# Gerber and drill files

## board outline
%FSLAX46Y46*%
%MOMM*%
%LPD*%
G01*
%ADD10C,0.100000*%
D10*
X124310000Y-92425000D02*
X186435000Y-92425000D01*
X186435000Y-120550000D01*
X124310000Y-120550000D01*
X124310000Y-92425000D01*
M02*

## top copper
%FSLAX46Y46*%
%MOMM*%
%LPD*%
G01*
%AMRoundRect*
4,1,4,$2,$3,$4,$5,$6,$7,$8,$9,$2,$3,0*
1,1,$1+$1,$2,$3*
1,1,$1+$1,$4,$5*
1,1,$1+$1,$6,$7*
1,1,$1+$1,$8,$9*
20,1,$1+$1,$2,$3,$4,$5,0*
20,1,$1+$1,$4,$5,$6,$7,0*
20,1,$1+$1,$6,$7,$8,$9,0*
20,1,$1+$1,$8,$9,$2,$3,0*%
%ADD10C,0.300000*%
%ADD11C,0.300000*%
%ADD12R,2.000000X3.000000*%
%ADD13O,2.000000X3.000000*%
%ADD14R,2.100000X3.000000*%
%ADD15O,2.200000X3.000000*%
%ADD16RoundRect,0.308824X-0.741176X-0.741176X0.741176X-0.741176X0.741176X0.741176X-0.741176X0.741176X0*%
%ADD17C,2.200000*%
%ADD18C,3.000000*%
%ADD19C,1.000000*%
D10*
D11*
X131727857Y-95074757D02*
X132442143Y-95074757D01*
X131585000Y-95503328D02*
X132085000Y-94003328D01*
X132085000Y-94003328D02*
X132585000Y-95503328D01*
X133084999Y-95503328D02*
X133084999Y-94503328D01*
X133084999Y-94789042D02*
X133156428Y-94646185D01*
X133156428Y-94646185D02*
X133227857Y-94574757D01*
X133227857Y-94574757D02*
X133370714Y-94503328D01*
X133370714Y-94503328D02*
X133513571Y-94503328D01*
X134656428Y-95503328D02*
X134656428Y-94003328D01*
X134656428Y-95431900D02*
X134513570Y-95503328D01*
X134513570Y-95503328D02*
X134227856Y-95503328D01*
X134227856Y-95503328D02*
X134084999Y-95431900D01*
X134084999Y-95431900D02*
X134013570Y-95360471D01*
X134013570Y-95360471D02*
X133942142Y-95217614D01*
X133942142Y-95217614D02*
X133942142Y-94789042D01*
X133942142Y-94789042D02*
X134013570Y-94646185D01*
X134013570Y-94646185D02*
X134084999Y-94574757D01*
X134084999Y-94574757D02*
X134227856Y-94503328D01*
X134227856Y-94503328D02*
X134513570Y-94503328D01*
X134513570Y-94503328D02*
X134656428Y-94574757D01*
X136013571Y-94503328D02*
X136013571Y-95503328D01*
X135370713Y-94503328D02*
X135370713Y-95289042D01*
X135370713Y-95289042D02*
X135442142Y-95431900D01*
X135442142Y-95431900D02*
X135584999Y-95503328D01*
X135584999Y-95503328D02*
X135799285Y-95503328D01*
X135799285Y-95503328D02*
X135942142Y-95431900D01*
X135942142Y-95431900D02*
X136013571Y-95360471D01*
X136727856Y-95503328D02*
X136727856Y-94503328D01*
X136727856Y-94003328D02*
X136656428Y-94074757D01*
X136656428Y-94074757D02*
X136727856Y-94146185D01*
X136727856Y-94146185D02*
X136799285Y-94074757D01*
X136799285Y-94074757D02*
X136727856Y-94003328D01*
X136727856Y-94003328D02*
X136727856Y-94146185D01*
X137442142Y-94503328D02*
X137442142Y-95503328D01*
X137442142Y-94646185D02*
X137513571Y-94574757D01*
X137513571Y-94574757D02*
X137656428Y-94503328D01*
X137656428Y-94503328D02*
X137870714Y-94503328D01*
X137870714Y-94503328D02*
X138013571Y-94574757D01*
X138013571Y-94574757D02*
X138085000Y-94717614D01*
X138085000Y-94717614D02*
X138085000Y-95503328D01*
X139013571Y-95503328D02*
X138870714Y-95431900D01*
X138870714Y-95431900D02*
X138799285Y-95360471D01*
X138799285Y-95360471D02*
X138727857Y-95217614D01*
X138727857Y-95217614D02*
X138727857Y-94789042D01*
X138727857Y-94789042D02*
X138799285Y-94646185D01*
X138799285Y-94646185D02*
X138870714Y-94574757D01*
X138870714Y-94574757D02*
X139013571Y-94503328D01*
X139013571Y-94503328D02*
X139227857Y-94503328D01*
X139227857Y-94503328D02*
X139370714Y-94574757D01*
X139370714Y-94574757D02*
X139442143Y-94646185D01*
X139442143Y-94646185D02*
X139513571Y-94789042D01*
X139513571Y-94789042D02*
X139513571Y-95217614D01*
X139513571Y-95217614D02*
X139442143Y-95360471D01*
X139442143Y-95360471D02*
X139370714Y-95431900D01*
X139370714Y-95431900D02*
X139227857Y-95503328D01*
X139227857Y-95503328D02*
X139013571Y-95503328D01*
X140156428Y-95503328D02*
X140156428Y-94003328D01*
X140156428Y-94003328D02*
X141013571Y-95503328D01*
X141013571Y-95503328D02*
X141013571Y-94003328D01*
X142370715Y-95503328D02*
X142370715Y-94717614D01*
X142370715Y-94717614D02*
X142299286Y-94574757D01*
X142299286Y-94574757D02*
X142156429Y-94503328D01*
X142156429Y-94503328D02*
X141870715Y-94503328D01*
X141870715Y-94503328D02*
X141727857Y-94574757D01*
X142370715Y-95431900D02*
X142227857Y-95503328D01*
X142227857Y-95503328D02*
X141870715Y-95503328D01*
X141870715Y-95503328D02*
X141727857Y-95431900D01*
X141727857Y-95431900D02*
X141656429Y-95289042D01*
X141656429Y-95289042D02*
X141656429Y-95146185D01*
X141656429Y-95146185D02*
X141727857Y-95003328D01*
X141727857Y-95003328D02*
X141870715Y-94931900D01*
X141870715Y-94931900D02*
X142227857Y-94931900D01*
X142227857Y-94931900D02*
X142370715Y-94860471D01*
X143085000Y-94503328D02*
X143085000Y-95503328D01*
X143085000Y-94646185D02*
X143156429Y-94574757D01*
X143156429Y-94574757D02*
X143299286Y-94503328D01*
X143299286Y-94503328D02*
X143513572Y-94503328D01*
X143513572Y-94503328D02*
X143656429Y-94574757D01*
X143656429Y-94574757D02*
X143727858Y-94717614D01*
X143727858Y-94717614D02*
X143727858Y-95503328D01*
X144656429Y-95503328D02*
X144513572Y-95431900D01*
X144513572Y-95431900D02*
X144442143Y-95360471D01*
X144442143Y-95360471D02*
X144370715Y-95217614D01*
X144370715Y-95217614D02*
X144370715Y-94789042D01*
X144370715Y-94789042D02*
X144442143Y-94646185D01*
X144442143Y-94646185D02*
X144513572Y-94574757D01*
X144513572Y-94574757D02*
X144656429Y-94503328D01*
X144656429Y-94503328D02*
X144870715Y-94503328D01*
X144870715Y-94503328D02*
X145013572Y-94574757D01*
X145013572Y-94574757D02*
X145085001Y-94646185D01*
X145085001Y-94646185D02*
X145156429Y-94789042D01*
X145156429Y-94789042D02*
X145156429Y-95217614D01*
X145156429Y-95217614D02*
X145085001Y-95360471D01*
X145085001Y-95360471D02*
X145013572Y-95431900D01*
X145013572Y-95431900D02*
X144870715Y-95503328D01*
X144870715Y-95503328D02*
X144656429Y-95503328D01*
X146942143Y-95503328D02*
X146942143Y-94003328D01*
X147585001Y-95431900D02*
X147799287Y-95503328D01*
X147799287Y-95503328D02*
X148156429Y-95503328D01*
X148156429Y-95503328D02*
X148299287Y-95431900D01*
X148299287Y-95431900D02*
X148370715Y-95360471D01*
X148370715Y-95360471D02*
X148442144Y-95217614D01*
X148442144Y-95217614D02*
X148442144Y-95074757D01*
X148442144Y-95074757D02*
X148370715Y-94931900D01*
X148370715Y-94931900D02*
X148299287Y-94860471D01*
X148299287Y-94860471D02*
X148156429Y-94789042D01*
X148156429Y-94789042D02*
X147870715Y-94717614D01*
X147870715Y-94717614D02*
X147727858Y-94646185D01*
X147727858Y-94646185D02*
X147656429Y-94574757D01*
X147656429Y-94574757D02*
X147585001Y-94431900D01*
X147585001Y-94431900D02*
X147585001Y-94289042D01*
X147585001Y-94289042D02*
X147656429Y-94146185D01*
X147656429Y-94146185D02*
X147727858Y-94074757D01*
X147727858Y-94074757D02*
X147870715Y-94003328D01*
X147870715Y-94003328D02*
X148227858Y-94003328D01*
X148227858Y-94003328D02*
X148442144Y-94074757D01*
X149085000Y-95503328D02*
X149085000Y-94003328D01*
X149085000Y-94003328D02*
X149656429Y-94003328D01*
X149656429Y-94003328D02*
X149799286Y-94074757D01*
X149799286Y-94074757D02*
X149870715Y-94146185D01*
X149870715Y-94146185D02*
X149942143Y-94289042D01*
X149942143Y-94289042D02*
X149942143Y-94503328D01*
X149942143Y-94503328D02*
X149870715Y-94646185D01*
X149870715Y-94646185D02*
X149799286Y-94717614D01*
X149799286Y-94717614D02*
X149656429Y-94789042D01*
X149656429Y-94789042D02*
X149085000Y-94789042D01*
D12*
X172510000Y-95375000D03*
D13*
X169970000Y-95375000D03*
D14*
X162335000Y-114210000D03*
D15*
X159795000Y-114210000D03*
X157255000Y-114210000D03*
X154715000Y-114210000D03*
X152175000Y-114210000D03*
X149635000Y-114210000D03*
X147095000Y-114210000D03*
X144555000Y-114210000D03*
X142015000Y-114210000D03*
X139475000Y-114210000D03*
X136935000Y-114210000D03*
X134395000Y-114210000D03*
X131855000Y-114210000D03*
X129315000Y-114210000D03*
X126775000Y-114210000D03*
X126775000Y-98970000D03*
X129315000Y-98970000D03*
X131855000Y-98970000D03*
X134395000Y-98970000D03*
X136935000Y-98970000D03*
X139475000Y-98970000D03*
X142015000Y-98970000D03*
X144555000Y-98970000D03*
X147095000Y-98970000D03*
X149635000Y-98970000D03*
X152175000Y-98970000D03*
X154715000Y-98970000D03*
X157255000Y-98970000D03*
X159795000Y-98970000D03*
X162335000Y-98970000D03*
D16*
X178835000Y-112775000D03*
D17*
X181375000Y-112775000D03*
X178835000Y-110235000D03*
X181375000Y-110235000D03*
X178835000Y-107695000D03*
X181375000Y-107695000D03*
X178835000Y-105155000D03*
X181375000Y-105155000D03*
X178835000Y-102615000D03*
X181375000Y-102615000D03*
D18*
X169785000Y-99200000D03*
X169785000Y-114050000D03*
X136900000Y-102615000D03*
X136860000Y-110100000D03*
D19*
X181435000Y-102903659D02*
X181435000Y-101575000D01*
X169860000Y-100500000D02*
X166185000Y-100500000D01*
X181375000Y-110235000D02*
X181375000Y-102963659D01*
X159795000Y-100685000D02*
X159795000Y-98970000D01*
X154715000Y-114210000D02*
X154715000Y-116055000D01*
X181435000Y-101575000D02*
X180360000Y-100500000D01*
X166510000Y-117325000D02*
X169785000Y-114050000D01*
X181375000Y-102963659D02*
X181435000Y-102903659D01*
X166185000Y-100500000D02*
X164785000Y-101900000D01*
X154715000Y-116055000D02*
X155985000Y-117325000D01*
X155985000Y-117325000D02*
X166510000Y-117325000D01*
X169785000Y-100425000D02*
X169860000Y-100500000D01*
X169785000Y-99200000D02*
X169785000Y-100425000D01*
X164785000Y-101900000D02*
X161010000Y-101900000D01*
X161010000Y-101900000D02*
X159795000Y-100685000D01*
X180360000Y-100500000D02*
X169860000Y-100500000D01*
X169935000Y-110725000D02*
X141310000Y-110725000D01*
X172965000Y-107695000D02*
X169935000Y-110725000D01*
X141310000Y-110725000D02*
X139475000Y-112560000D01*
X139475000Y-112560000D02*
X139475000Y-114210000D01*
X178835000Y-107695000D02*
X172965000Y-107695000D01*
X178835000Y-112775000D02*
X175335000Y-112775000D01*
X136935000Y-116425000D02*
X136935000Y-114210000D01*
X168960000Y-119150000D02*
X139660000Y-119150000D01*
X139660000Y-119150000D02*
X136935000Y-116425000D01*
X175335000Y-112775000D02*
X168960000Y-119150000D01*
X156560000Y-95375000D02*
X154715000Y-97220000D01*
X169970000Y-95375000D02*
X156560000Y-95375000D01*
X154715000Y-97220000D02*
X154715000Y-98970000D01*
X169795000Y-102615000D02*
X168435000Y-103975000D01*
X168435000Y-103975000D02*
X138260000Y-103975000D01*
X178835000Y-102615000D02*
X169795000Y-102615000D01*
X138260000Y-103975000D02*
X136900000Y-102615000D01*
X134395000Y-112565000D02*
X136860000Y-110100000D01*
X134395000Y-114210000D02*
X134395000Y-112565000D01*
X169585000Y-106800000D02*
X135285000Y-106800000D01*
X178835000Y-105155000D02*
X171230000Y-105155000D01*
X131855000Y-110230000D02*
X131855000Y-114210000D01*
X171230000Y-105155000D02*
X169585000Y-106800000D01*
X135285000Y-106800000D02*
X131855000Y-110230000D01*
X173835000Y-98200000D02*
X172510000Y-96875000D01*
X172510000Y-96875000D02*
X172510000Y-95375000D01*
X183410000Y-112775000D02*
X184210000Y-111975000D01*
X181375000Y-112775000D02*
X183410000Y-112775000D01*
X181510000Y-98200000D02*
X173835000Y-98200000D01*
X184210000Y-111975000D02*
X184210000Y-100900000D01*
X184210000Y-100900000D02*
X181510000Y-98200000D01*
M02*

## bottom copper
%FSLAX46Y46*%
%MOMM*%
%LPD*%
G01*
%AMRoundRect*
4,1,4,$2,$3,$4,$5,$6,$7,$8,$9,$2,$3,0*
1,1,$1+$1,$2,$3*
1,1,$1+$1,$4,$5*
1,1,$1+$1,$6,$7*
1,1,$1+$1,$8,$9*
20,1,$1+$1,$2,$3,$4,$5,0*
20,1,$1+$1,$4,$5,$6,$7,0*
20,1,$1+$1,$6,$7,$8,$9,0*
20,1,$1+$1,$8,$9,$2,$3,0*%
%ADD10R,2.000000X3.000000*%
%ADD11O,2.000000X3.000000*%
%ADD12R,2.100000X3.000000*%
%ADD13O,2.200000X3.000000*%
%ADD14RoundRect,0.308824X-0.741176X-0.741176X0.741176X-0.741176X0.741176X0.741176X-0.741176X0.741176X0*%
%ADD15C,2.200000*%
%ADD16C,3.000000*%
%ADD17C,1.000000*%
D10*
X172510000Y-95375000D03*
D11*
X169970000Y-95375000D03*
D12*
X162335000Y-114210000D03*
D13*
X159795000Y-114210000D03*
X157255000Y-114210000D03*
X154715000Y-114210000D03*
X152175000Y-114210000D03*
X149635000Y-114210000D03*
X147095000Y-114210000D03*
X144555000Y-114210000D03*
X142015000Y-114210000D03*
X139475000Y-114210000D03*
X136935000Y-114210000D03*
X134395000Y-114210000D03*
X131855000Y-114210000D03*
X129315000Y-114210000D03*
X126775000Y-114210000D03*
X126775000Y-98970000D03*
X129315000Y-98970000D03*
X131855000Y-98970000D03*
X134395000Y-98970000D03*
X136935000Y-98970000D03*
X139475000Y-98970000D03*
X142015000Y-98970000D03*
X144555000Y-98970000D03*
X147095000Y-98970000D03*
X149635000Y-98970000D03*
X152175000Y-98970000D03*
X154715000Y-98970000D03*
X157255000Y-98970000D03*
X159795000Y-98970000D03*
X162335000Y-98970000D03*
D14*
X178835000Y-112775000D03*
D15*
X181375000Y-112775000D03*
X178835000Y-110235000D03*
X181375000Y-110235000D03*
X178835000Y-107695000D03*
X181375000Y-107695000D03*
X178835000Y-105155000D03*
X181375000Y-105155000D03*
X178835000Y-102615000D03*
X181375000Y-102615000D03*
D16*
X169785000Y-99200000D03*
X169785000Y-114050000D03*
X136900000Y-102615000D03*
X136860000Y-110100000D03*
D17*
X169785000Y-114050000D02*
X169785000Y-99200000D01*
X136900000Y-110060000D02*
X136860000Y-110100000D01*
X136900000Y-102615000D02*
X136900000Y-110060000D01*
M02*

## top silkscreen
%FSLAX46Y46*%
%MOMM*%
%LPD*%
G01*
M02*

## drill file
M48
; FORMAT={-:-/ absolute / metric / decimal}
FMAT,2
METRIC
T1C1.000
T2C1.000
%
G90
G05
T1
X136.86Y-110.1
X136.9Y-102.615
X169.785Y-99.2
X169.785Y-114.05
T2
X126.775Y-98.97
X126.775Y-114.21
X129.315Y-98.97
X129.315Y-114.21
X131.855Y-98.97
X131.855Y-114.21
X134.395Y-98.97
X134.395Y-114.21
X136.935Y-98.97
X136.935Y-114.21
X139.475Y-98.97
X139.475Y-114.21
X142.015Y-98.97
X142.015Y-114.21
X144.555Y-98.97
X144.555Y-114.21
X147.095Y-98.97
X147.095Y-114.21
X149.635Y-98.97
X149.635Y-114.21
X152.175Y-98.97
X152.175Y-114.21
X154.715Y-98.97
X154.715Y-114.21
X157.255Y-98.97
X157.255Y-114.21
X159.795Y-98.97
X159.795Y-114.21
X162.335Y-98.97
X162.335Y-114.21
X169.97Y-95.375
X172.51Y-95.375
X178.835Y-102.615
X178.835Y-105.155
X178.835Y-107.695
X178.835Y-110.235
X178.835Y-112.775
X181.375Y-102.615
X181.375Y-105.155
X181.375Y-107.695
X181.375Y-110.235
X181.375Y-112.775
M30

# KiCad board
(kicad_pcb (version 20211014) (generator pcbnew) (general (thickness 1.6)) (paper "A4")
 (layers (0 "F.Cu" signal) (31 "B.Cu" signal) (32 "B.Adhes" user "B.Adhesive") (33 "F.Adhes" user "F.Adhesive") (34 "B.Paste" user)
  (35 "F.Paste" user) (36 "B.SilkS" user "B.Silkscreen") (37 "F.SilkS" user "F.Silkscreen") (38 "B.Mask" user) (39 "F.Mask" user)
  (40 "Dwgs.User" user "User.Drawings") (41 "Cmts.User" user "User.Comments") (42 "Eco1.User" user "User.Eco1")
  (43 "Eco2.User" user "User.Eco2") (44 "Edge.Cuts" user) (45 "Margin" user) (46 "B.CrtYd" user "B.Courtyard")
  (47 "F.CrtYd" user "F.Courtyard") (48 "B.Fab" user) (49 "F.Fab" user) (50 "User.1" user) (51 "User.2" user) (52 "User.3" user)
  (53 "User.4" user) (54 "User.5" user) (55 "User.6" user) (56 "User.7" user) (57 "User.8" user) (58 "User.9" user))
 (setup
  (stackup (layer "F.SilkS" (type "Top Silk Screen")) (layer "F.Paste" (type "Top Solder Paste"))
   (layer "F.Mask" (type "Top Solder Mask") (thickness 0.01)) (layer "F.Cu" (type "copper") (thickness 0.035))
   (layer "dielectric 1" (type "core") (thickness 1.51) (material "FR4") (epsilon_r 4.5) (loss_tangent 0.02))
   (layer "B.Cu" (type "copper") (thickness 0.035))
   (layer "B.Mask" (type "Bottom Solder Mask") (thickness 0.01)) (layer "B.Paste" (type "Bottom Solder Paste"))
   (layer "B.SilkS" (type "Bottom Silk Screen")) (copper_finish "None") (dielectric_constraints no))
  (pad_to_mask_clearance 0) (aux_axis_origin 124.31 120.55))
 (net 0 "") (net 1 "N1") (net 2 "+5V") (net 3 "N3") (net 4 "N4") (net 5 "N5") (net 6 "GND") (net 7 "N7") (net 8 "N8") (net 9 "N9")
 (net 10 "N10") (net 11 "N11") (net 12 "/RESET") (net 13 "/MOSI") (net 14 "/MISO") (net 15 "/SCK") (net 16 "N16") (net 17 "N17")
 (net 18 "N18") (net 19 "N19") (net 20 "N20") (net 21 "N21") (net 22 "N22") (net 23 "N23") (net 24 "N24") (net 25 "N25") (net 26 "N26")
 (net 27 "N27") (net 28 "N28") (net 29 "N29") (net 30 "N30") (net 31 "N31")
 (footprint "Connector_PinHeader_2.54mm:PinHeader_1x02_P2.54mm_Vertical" (layer "B.Cu") (at 172.51 95.375 90)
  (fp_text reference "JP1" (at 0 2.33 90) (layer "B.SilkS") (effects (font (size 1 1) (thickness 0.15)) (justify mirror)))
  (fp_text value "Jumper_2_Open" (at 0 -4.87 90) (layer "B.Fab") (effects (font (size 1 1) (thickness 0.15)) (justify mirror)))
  (pad "1" thru_hole rect locked (at 0 0 90) (size 3 2) (drill 1) (layers *.Cu *.Mask) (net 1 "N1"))
  (pad "2" thru_hole oval locked (at 0 -2.54 90) (size 3 2) (drill 1) (layers *.Cu *.Mask) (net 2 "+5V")))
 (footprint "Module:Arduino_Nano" (layer "B.Cu") (at 162.335 114.21 90)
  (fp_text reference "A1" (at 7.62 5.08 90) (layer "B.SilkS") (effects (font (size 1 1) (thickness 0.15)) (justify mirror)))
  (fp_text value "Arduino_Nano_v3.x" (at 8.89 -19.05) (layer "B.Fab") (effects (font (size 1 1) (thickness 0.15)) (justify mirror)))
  (pad "1" thru_hole rect locked (at 0 0 90) (size 3 2.1) (drill 1) (layers *.Cu *.Mask) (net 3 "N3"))
  (pad "2" thru_hole oval locked (at 0 -2.54 90) (size 3 2.2) (drill 1) (layers *.Cu *.Mask) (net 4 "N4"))
  (pad "3" thru_hole oval locked (at 0 -5.08 90) (size 3 2.2) (drill 1) (layers *.Cu *.Mask) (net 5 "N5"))
  (pad "4" thru_hole oval locked (at 0 -7.62 90) (size 3 2.2) (drill 1) (layers *.Cu *.Mask) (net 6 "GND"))
  (pad "5" thru_hole oval locked (at 0 -10.16 90) (size 3 2.2) (drill 1) (layers *.Cu *.Mask) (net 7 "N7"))
  (pad "6" thru_hole oval locked (at 0 -12.7 90) (size 3 2.2) (drill 1) (layers *.Cu *.Mask) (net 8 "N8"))
  (pad "7" thru_hole oval locked (at 0 -15.24 90) (size 3 2.2) (drill 1) (layers *.Cu *.Mask) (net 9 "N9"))
  (pad "8" thru_hole oval locked (at 0 -17.78 90) (size 3 2.2) (drill 1) (layers *.Cu *.Mask) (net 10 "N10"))
  (pad "9" thru_hole oval locked (at 0 -20.32 90) (size 3 2.2) (drill 1) (layers *.Cu *.Mask) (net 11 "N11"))
  (pad "10" thru_hole oval locked (at 0 -22.86 90) (size 3 2.2) (drill 1) (layers *.Cu *.Mask) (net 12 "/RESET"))
  (pad "11" thru_hole oval locked (at 0 -25.4 90) (size 3 2.2) (drill 1) (layers *.Cu *.Mask) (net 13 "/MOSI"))
  (pad "12" thru_hole oval locked (at 0 -27.94 90) (size 3 2.2) (drill 1) (layers *.Cu *.Mask) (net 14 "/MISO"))
  (pad "13" thru_hole oval locked (at 0 -30.48 90) (size 3 2.2) (drill 1) (layers *.Cu *.Mask) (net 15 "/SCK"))
  (pad "14" thru_hole oval locked (at 0 -33.02 90) (size 3 2.2) (drill 1) (layers *.Cu *.Mask) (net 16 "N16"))
  (pad "15" thru_hole oval locked (at 0 -35.56 90) (size 3 2.2) (drill 1) (layers *.Cu *.Mask) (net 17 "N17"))
  (pad "16" thru_hole oval locked (at 15.24 -35.56 90) (size 3 2.2) (drill 1) (layers *.Cu *.Mask) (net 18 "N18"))
  (pad "17" thru_hole oval locked (at 15.24 -33.02 90) (size 3 2.2) (drill 1) (layers *.Cu *.Mask) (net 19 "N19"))
  (pad "18" thru_hole oval locked (at 15.24 -30.48 90) (size 3 2.2) (drill 1) (layers *.Cu *.Mask) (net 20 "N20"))
  (pad "19" thru_hole oval locked (at 15.24 -27.94 90) (size 3 2.2) (drill 1) (layers *.Cu *.Mask) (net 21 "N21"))
  (pad "20" thru_hole oval locked (at 15.24 -25.4 90) (size 3 2.2) (drill 1) (layers *.Cu *.Mask) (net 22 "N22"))
  (pad "21" thru_hole oval locked (at 15.24 -22.86 90) (size 3 2.2) (drill 1) (layers *.Cu *.Mask) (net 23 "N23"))
  (pad "22" thru_hole oval locked (at 15.24 -20.32 90) (size 3 2.2) (drill 1) (layers *.Cu *.Mask) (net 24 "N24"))
  (pad "23" thru_hole oval locked (at 15.24 -17.78 90) (size 3 2.2) (drill 1) (layers *.Cu *.Mask) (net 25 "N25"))
  (pad "24" thru_hole oval locked (at 15.24 -15.24 90) (size 3 2.2) (drill 1) (layers *.Cu *.Mask) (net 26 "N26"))
  (pad "25" thru_hole oval locked (at 15.24 -12.7 90) (size 3 2.2) (drill 1) (layers *.Cu *.Mask) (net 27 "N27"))
  (pad "26" thru_hole oval locked (at 15.24 -10.16 90) (size 3 2.2) (drill 1) (layers *.Cu *.Mask) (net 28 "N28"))
  (pad "27" thru_hole oval locked (at 15.24 -7.62 90) (size 3 2.2) (drill 1) (layers *.Cu *.Mask) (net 2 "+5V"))
  (pad "28" thru_hole oval locked (at 15.24 -5.08 90) (size 3 2.2) (drill 1) (layers *.Cu *.Mask) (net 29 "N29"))
  (pad "29" thru_hole oval locked (at 15.24 -2.54 90) (size 3 2.2) (drill 1) (layers *.Cu *.Mask) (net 6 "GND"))
  (pad "30" thru_hole oval locked (at 15.24 0 90) (size 3 2.2) (drill 1) (layers *.Cu *.Mask) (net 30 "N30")))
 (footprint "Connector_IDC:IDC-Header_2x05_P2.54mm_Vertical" (layer "B.Cu") (at 178.835 112.775)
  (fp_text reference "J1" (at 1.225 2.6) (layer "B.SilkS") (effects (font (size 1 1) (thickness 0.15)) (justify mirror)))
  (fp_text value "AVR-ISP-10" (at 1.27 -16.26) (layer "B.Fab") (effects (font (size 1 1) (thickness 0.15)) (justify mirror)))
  (pad "1" thru_hole roundrect locked (at 0 0) (size 2.1 2.1) (drill 1) (layers *.Cu *.Mask) (roundrect_rratio 0.1470590476)
   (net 13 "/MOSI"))
  (pad "2" thru_hole circle locked (at 2.54 0) (size 2.2 2.2) (drill 1) (layers *.Cu *.Mask) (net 1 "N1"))
  (pad "3" thru_hole circle locked (at 0 -2.54) (size 2.2 2.2) (drill 1) (layers *.Cu *.Mask) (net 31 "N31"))
  (pad "4" thru_hole circle locked (at 2.54 -2.54) (size 2.2 2.2) (drill 1) (layers *.Cu *.Mask) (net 6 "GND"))
  (pad "5" thru_hole circle locked (at 0 -5.08) (size 2.2 2.2) (drill 1) (layers *.Cu *.Mask) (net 12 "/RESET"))
  (pad "6" thru_hole circle locked (at 2.54 -5.08) (size 2.2 2.2) (drill 1) (layers *.Cu *.Mask) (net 6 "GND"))
  (pad "7" thru_hole circle locked (at 0 -7.62) (size 2.2 2.2) (drill 1) (layers *.Cu *.Mask) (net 15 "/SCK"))
  (pad "8" thru_hole circle locked (at 2.54 -7.62) (size 2.2 2.2) (drill 1) (layers *.Cu *.Mask) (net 6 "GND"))
  (pad "9" thru_hole circle locked (at 0 -10.16) (size 2.2 2.2) (drill 1) (layers *.Cu *.Mask) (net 14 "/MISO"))
  (pad "10" thru_hole circle locked (at 2.54 -10.16) (size 2.2 2.2) (drill 1) (layers *.Cu *.Mask) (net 6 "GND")))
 (gr_rect (start 124.31 120.55) (end 186.435 92.425) (layer "Edge.Cuts") (width 0.1) (fill none))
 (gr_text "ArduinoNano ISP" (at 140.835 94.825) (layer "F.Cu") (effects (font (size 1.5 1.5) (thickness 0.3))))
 (segment (start 181.435 102.903659) (end 181.435 101.575) (width 1) (layer "F.Cu") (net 6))
 (segment (start 169.86 100.5) (end 166.185 100.5) (width 1) (layer "F.Cu") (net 6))
 (segment (start 181.375 110.235) (end 181.375 102.963659) (width 1) (layer "F.Cu") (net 6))
 (segment (start 159.795 100.685) (end 159.795 98.97) (width 1) (layer "F.Cu") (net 6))
 (segment (start 154.715 114.21) (end 154.715 116.055) (width 1) (layer "F.Cu") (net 6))
 (segment (start 181.435 101.575) (end 180.36 100.5) (width 1) (layer "F.Cu") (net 6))
 (segment (start 166.51 117.325) (end 169.785 114.05) (width 1) (layer "F.Cu") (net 6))
 (segment (start 181.375 102.963659) (end 181.435 102.903659) (width 1) (layer "F.Cu") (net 6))
 (segment (start 166.185 100.5) (end 164.785 101.9) (width 1) (layer "F.Cu") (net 6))
 (segment (start 154.715 116.055) (end 155.985 117.325) (width 1) (layer "F.Cu") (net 6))
 (segment (start 155.985 117.325) (end 166.51 117.325) (width 1) (layer "F.Cu") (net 6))
 (segment (start 169.785 100.425) (end 169.86 100.5) (width 1) (layer "F.Cu") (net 6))
 (segment (start 169.785 99.2) (end 169.785 100.425) (width 1) (layer "F.Cu") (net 6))
 (segment (start 164.785 101.9) (end 161.01 101.9) (width 1) (layer "F.Cu") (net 6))
 (segment (start 161.01 101.9) (end 159.795 100.685) (width 1) (layer "F.Cu") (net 6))
 (segment (start 180.36 100.5) (end 169.86 100.5) (width 1) (layer "F.Cu") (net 6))
 (via (at 169.785 99.2) (size 3) (drill 1) (layers "F.Cu" "B.Cu") (free) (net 6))
 (via (at 169.785 114.05) (size 3) (drill 1) (layers "F.Cu" "B.Cu") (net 6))
 (segment (start 169.785 114.05) (end 169.785 99.2) (width 1) (layer "B.Cu") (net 6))
 (segment (start 169.935 110.725) (end 141.31 110.725) (width 1) (layer "F.Cu") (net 12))
 (segment (start 172.965 107.695) (end 169.935 110.725) (width 1) (layer "F.Cu") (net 12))
 (segment (start 141.31 110.725) (end 139.475 112.56) (width 1) (layer "F.Cu") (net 12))
 (segment (start 139.475 112.56) (end 139.475 114.21) (width 1) (layer "F.Cu") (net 12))
 (segment (start 178.835 107.695) (end 172.965 107.695) (width 1) (layer "F.Cu") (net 12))
 (segment (start 178.835 112.775) (end 175.335 112.775) (width 1) (layer "F.Cu") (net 13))
 (segment (start 136.935 116.425) (end 136.935 114.21) (width 1) (layer "F.Cu") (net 13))
 (segment (start 168.96 119.15) (end 139.66 119.15) (width 1) (layer "F.Cu") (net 13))
 (segment (start 139.66 119.15) (end 136.935 116.425) (width 1) (layer "F.Cu") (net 13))
 (segment (start 175.335 112.775) (end 168.96 119.15) (width 1) (layer "F.Cu") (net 13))
 (segment (start 156.56 95.375) (end 154.715 97.22) (width 1) (layer "F.Cu") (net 2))
 (segment (start 169.97 95.375) (end 156.56 95.375) (width 1) (layer "F.Cu") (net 2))
 (segment (start 154.715 97.22) (end 154.715 98.97) (width 1) (layer "F.Cu") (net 2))
 (segment (start 169.795 102.615) (end 168.435 103.975) (width 1) (layer "F.Cu") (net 14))
 (segment (start 168.435 103.975) (end 138.26 103.975) (width 1) (layer "F.Cu") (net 14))
 (segment (start 178.835 102.615) (end 169.795 102.615) (width 1) (layer "F.Cu") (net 14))
 (segment (start 138.26 103.975) (end 136.9 102.615) (width 1) (layer "F.Cu") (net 14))
 (segment (start 134.395 112.565) (end 136.86 110.1) (width 1) (layer "F.Cu") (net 14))
 (segment (start 134.395 114.21) (end 134.395 112.565) (width 1) (layer "F.Cu") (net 14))
 (via (at 136.9 102.615) (size 3) (drill 1) (layers "F.Cu" "B.Cu") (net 14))
 (via (at 136.86 110.1) (size 3) (drill 1) (layers "F.Cu" "B.Cu") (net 14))
 (segment (start 136.9 110.06) (end 136.86 110.1) (width 1) (layer "B.Cu") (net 14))
 (segment (start 136.9 102.615) (end 136.9 110.06) (width 1) (layer "B.Cu") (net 14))
 (segment (start 169.585 106.8) (end 135.285 106.8) (width 1) (layer "F.Cu") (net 15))
 (segment (start 178.835 105.155) (end 171.23 105.155) (width 1) (layer "F.Cu") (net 15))
 (segment (start 131.855 110.23) (end 131.855 114.21) (width 1) (layer "F.Cu") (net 15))
 (segment (start 171.23 105.155) (end 169.585 106.8) (width 1) (layer "F.Cu") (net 15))
 (segment (start 135.285 106.8) (end 131.855 110.23) (width 1) (layer "F.Cu") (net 15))
 (segment (start 173.835 98.2) (end 172.51 96.875) (width 1) (layer "F.Cu") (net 1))
 (segment (start 172.51 96.875) (end 172.51 95.375) (width 1) (layer "F.Cu") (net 1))
 (segment (start 183.41 112.775) (end 184.21 111.975) (width 1) (layer "F.Cu") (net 1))
 (segment (start 181.375 112.775) (end 183.41 112.775) (width 1) (layer "F.Cu") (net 1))
 (segment (start 181.51 98.2) (end 173.835 98.2) (width 1) (layer "F.Cu") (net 1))
 (segment (start 184.21 111.975) (end 184.21 100.9) (width 1) (layer "F.Cu") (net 1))
 (segment (start 184.21 100.9) (end 181.51 98.2) (width 1) (layer "F.Cu") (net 1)))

